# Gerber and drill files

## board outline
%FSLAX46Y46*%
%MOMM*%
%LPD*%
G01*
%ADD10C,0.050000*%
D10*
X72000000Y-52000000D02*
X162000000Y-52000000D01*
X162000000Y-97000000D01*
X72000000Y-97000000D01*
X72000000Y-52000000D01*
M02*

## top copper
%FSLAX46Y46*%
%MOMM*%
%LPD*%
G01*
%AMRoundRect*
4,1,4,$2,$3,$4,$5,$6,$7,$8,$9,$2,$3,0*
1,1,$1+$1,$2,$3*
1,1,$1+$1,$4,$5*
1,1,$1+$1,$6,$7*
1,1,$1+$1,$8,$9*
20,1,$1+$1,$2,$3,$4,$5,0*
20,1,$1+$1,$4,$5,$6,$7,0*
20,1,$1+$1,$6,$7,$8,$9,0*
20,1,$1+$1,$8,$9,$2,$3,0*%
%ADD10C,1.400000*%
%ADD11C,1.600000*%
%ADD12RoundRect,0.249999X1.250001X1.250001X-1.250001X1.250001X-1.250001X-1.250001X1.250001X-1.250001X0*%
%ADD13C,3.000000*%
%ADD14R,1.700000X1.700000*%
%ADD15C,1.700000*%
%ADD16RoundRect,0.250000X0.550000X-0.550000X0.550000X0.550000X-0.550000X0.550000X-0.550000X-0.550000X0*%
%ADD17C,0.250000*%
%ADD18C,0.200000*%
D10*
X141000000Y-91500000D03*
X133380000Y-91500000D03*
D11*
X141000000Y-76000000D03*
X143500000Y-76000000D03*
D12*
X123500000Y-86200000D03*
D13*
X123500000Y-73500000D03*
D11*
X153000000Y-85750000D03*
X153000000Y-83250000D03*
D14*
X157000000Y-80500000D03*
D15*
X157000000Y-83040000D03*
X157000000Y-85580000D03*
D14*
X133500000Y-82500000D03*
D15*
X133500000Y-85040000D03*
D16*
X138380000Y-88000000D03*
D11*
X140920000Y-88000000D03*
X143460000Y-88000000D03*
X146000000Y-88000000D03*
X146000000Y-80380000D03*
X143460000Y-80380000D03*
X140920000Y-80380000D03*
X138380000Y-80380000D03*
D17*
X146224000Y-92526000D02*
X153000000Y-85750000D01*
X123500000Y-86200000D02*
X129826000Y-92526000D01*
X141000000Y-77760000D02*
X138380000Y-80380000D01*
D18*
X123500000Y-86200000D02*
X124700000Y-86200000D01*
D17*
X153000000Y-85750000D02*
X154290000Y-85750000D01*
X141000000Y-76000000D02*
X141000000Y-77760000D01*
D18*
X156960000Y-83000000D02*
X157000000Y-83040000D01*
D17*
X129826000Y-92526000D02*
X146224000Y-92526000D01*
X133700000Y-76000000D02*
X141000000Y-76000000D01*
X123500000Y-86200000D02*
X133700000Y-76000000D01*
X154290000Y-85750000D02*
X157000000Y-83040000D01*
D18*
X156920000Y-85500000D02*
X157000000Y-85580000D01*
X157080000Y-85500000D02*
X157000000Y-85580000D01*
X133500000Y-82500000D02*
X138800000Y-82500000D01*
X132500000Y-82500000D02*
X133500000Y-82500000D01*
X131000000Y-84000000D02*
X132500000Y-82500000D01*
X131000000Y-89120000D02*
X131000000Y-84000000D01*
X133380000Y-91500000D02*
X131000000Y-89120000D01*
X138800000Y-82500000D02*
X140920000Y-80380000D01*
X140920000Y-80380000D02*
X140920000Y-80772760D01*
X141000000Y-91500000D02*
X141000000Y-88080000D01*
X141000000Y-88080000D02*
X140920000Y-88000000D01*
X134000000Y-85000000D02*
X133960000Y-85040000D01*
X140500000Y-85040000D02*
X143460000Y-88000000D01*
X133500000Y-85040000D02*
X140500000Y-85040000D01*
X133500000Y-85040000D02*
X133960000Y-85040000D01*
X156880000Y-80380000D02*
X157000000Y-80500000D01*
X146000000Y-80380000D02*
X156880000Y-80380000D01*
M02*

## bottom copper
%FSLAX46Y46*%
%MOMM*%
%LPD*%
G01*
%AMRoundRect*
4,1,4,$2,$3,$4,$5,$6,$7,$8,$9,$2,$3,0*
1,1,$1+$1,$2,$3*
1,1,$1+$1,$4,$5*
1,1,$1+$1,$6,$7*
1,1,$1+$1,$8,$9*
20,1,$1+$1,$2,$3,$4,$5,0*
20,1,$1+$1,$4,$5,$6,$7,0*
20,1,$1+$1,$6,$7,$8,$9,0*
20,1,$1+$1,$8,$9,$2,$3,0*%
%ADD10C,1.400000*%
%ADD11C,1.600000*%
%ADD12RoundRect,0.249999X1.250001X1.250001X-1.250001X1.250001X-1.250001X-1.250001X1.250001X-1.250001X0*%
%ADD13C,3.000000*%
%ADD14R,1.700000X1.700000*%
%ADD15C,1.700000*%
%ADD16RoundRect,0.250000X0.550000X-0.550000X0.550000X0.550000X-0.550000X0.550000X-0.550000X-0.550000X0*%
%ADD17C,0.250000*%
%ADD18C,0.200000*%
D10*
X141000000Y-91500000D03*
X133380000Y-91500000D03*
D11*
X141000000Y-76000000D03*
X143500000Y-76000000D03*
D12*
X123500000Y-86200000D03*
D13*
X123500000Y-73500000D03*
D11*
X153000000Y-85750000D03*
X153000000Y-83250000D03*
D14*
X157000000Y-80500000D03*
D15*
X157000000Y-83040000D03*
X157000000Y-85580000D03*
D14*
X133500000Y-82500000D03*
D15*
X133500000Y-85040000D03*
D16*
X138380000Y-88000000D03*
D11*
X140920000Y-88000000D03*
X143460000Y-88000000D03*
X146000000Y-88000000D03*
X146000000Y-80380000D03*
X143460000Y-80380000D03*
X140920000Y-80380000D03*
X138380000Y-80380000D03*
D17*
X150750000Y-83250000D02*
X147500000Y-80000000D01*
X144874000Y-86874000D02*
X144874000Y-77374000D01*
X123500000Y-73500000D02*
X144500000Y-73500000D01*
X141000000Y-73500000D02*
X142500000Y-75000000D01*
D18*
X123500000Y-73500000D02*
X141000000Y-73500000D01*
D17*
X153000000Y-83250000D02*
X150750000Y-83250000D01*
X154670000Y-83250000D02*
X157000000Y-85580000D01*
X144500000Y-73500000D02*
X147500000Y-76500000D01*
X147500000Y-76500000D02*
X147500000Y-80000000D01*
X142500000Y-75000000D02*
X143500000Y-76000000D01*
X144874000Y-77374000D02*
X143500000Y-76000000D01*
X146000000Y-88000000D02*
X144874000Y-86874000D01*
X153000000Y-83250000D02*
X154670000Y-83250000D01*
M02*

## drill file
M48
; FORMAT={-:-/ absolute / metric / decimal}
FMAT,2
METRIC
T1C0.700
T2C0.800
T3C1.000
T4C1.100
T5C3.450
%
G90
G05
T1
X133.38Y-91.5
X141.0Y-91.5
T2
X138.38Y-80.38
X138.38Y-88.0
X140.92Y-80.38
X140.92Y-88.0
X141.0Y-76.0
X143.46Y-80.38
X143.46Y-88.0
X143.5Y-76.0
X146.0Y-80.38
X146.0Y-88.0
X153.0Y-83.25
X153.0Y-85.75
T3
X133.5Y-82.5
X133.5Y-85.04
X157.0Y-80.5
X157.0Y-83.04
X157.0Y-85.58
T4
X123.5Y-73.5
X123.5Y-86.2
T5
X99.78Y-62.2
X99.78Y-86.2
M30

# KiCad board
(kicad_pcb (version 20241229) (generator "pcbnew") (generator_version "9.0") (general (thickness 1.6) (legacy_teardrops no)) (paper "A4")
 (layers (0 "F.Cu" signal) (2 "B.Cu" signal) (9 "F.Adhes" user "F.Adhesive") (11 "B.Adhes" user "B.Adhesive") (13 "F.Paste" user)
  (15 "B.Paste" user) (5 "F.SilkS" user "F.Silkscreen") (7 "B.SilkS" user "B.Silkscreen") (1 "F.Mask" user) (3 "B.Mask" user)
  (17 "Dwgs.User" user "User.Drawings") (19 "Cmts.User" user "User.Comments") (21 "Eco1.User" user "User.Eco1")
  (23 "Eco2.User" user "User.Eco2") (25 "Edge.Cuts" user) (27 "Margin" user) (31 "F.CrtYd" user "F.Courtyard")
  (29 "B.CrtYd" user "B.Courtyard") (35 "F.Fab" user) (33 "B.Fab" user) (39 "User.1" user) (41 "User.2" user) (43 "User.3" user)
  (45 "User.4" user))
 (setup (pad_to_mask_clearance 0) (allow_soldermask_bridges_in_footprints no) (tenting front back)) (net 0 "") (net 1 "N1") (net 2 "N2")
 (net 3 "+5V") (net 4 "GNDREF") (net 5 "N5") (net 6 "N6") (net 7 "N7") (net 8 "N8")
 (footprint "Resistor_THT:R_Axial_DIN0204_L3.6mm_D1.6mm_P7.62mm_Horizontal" (layer "F.Cu") (at 141 91.5 180)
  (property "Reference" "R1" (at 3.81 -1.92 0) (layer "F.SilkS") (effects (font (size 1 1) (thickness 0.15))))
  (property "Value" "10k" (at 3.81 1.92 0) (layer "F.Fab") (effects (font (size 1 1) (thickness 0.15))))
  (pad "1" thru_hole circle (at 0 0 180) (size 1.4 1.4) (drill 0.7) (layers "*.Cu" "*.Mask") (remove_unused_layers no) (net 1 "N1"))
  (pad "2" thru_hole circle (at 7.62 0 180) (size 1.4 1.4) (drill 0.7) (layers "*.Cu" "*.Mask") (remove_unused_layers no) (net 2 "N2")))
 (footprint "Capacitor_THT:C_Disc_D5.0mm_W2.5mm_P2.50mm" (layer "F.Cu") (at 141 76)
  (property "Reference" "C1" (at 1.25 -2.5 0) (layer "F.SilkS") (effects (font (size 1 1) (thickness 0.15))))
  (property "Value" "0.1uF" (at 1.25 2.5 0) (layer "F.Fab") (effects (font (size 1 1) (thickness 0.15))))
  (pad "1" thru_hole circle (at 0 0) (size 1.6 1.6) (drill 0.8) (layers "*.Cu" "*.Mask") (remove_unused_layers no) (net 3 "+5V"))
  (pad "2" thru_hole circle (at 2.5 0) (size 1.6 1.6) (drill 0.8) (layers "*.Cu" "*.Mask") (remove_unused_layers no) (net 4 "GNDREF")))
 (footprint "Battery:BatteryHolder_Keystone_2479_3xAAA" (layer "F.Cu") (at 123.5 86.2 180)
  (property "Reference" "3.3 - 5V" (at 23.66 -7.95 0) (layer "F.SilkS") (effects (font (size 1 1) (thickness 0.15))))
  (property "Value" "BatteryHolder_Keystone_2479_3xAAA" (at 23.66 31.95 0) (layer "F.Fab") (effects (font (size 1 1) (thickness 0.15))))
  (pad "" np_thru_hole circle (at 23.72 0 180) (size 3.45 3.45) (drill 3.45) (layers "*.Cu" "*.Mask"))
  (pad "" np_thru_hole circle (at 23.72 24 180) (size 3.45 3.45) (drill 3.45) (layers "*.Cu" "*.Mask"))
  (pad "1" thru_hole roundrect (at 0 0 180) (size 3 3) (drill 1.1) (layers "*.Cu" "*.Mask") (remove_unused_layers no)
   (roundrect_rratio 0.083333) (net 3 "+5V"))
  (pad "2" thru_hole circle (at 0 12.7 180) (size 3 3) (drill 1.1) (layers "*.Cu" "*.Mask") (remove_unused_layers no) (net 4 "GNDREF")))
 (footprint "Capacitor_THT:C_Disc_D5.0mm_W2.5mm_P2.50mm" (layer "F.Cu") (at 153 85.75 90)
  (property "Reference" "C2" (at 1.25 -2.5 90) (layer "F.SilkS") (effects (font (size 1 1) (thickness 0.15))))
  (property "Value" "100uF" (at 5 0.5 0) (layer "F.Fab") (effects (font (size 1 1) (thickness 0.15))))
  (pad "1" thru_hole circle (at 0 0 90) (size 1.6 1.6) (drill 0.8) (layers "*.Cu" "*.Mask") (remove_unused_layers no) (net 3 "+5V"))
  (pad "2" thru_hole circle (at 2.5 0 90) (size 1.6 1.6) (drill 0.8) (layers "*.Cu" "*.Mask") (remove_unused_layers no) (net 4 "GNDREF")))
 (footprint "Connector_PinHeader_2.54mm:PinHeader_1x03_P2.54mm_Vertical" (layer "F.Cu") (at 157 80.5)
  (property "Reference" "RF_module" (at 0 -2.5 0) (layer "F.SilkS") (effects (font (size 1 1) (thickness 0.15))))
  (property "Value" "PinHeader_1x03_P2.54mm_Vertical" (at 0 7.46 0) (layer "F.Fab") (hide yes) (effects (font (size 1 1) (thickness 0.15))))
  (pad "1" thru_hole rect (at 0 0) (size 1.7 1.7) (drill 1) (layers "*.Cu" "*.Mask") (remove_unused_layers no) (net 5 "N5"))
  (pad "2" thru_hole circle (at 0 2.54) (size 1.7 1.7) (drill 1) (layers "*.Cu" "*.Mask") (remove_unused_layers no) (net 3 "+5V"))
  (pad "3" thru_hole circle (at 0 5.08) (size 1.7 1.7) (drill 1) (layers "*.Cu" "*.Mask") (remove_unused_layers no) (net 4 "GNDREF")))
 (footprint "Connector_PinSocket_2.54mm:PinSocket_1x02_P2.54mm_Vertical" (layer "F.Cu") (at 133.5 82.5)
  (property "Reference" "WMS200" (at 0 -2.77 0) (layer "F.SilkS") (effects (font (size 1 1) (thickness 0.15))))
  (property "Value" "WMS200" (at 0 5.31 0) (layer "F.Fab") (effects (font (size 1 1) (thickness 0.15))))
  (pad "1" thru_hole rect (at 0 0) (size 1.7 1.7) (drill 1) (layers "*.Cu" "*.Mask") (remove_unused_layers no) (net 2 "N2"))
  (pad "2" thru_hole circle (at 0 2.54) (size 1.7 1.7) (drill 1) (layers "*.Cu" "*.Mask") (remove_unused_layers no) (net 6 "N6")))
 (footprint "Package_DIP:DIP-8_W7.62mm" (layer "F.Cu") (at 138.38 88 90)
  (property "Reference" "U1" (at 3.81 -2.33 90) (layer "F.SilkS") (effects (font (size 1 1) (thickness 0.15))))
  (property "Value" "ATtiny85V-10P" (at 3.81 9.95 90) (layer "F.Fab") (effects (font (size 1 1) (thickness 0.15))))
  (pad "1" thru_hole roundrect (at 0 0 90) (size 1.6 1.6) (drill 0.8) (layers "*.Cu" "*.Mask") (remove_unused_layers no)
   (roundrect_rratio 0.15625) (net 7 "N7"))
  (pad "2" thru_hole circle (at 0 2.54 90) (size 1.6 1.6) (drill 0.8) (layers "*.Cu" "*.Mask") (remove_unused_layers no) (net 1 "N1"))
  (pad "3" thru_hole circle (at 0 5.08 90) (size 1.6 1.6) (drill 0.8) (layers "*.Cu" "*.Mask") (remove_unused_layers no) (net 6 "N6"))
  (pad "4" thru_hole circle (at 0 7.62 90) (size 1.6 1.6) (drill 0.8) (layers "*.Cu" "*.Mask") (remove_unused_layers no) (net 4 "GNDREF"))
  (pad "5" thru_hole circle (at 7.62 7.62 90) (size 1.6 1.6) (drill 0.8) (layers "*.Cu" "*.Mask") (remove_unused_layers no) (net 5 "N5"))
  (pad "6" thru_hole circle (at 7.62 5.08 90) (size 1.6 1.6) (drill 0.8) (layers "*.Cu" "*.Mask") (remove_unused_layers no) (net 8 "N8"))
  (pad "7" thru_hole circle (at 7.62 2.54 90) (size 1.6 1.6) (drill 0.8) (layers "*.Cu" "*.Mask") (remove_unused_layers no) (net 2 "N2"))
  (pad "8" thru_hole circle (at 7.62 0 90) (size 1.6 1.6) (drill 0.8) (layers "*.Cu" "*.Mask") (remove_unused_layers no) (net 3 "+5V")))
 (gr_rect (start 72 52) (end 162 97) (stroke (width 0.05) (type default)) (fill no) (layer "Edge.Cuts"))
 (segment (start 146.224 92.526) (end 153 85.75) (width 0.25) (layer "F.Cu") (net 3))
 (segment (start 123.5 86.2) (end 129.826 92.526) (width 0.25) (layer "F.Cu") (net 3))
 (segment (start 141 77.76) (end 138.38 80.38) (width 0.25) (layer "F.Cu") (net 3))
 (segment (start 123.5 86.2) (end 124.7 86.2) (width 0.2) (layer "F.Cu") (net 3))
 (segment (start 153 85.75) (end 154.29 85.75) (width 0.25) (layer "F.Cu") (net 3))
 (segment (start 141 76) (end 141 77.76) (width 0.25) (layer "F.Cu") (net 3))
 (segment (start 156.96 83) (end 157 83.04) (width 0.2) (layer "F.Cu") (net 3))
 (segment (start 129.826 92.526) (end 146.224 92.526) (width 0.25) (layer "F.Cu") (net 3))
 (segment (start 133.7 76) (end 141 76) (width 0.25) (layer "F.Cu") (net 3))
 (segment (start 123.5 86.2) (end 133.7 76) (width 0.25) (layer "F.Cu") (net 3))
 (segment (start 154.29 85.75) (end 157 83.04) (width 0.25) (layer "F.Cu") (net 3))
 (segment (start 156.92 85.5) (end 157 85.58) (width 0.2) (layer "F.Cu") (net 4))
 (segment (start 157.08 85.5) (end 157 85.58) (width 0.2) (layer "F.Cu") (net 4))
 (segment (start 150.75 83.25) (end 147.5 80) (width 0.25) (layer "B.Cu") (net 4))
 (segment (start 144.874 86.874) (end 144.874 77.374) (width 0.25) (layer "B.Cu") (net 4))
 (segment (start 123.5 73.5) (end 144.5 73.5) (width 0.25) (layer "B.Cu") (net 4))
 (segment (start 141 73.5) (end 142.5 75) (width 0.25) (layer "B.Cu") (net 4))
 (segment (start 123.5 73.5) (end 141 73.5) (width 0.2) (layer "B.Cu") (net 4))
 (segment (start 153 83.25) (end 150.75 83.25) (width 0.25) (layer "B.Cu") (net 4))
 (segment (start 154.67 83.25) (end 157 85.58) (width 0.25) (layer "B.Cu") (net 4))
 (segment (start 144.5 73.5) (end 147.5 76.5) (width 0.25) (layer "B.Cu") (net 4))
 (segment (start 147.5 76.5) (end 147.5 80) (width 0.25) (layer "B.Cu") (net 4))
 (segment (start 142.5 75) (end 143.5 76) (width 0.25) (layer "B.Cu") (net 4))
 (segment (start 144.874 77.374) (end 143.5 76) (width 0.25) (layer "B.Cu") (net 4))
 (segment (start 146 88) (end 144.874 86.874) (width 0.25) (layer "B.Cu") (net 4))
 (segment (start 153 83.25) (end 154.67 83.25) (width 0.25) (layer "B.Cu") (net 4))
 (segment (start 133.5 82.5) (end 138.8 82.5) (width 0.2) (layer "F.Cu") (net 2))
 (segment (start 132.5 82.5) (end 133.5 82.5) (width 0.2) (layer "F.Cu") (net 2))
 (segment (start 131 84) (end 132.5 82.5) (width 0.2) (layer "F.Cu") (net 2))
 (segment (start 131 89.12) (end 131 84) (width 0.2) (layer "F.Cu") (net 2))
 (segment (start 133.38 91.5) (end 131 89.12) (width 0.2) (layer "F.Cu") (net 2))
 (segment (start 138.8 82.5) (end 140.92 80.38) (width 0.2) (layer "F.Cu") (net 2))
 (segment (start 140.92 80.38) (end 140.92 80.77276) (width 0.2) (layer "F.Cu") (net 2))
 (segment (start 141 91.5) (end 141 88.08) (width 0.2) (layer "F.Cu") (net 1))
 (segment (start 141 88.08) (end 140.92 88) (width 0.2) (layer "F.Cu") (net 1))
 (segment (start 134 85) (end 133.96 85.04) (width 0.2) (layer "F.Cu") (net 6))
 (segment (start 140.5 85.04) (end 143.46 88) (width 0.2) (layer "F.Cu") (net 6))
 (segment (start 133.5 85.04) (end 140.5 85.04) (width 0.2) (layer "F.Cu") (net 6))
 (segment (start 133.5 85.04) (end 133.96 85.04) (width 0.2) (layer "F.Cu") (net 6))
 (segment (start 156.88 80.38) (end 157 80.5) (width 0.2) (layer "F.Cu") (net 5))
 (segment (start 146 80.38) (end 156.88 80.38) (width 0.2) (layer "F.Cu") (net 5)))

